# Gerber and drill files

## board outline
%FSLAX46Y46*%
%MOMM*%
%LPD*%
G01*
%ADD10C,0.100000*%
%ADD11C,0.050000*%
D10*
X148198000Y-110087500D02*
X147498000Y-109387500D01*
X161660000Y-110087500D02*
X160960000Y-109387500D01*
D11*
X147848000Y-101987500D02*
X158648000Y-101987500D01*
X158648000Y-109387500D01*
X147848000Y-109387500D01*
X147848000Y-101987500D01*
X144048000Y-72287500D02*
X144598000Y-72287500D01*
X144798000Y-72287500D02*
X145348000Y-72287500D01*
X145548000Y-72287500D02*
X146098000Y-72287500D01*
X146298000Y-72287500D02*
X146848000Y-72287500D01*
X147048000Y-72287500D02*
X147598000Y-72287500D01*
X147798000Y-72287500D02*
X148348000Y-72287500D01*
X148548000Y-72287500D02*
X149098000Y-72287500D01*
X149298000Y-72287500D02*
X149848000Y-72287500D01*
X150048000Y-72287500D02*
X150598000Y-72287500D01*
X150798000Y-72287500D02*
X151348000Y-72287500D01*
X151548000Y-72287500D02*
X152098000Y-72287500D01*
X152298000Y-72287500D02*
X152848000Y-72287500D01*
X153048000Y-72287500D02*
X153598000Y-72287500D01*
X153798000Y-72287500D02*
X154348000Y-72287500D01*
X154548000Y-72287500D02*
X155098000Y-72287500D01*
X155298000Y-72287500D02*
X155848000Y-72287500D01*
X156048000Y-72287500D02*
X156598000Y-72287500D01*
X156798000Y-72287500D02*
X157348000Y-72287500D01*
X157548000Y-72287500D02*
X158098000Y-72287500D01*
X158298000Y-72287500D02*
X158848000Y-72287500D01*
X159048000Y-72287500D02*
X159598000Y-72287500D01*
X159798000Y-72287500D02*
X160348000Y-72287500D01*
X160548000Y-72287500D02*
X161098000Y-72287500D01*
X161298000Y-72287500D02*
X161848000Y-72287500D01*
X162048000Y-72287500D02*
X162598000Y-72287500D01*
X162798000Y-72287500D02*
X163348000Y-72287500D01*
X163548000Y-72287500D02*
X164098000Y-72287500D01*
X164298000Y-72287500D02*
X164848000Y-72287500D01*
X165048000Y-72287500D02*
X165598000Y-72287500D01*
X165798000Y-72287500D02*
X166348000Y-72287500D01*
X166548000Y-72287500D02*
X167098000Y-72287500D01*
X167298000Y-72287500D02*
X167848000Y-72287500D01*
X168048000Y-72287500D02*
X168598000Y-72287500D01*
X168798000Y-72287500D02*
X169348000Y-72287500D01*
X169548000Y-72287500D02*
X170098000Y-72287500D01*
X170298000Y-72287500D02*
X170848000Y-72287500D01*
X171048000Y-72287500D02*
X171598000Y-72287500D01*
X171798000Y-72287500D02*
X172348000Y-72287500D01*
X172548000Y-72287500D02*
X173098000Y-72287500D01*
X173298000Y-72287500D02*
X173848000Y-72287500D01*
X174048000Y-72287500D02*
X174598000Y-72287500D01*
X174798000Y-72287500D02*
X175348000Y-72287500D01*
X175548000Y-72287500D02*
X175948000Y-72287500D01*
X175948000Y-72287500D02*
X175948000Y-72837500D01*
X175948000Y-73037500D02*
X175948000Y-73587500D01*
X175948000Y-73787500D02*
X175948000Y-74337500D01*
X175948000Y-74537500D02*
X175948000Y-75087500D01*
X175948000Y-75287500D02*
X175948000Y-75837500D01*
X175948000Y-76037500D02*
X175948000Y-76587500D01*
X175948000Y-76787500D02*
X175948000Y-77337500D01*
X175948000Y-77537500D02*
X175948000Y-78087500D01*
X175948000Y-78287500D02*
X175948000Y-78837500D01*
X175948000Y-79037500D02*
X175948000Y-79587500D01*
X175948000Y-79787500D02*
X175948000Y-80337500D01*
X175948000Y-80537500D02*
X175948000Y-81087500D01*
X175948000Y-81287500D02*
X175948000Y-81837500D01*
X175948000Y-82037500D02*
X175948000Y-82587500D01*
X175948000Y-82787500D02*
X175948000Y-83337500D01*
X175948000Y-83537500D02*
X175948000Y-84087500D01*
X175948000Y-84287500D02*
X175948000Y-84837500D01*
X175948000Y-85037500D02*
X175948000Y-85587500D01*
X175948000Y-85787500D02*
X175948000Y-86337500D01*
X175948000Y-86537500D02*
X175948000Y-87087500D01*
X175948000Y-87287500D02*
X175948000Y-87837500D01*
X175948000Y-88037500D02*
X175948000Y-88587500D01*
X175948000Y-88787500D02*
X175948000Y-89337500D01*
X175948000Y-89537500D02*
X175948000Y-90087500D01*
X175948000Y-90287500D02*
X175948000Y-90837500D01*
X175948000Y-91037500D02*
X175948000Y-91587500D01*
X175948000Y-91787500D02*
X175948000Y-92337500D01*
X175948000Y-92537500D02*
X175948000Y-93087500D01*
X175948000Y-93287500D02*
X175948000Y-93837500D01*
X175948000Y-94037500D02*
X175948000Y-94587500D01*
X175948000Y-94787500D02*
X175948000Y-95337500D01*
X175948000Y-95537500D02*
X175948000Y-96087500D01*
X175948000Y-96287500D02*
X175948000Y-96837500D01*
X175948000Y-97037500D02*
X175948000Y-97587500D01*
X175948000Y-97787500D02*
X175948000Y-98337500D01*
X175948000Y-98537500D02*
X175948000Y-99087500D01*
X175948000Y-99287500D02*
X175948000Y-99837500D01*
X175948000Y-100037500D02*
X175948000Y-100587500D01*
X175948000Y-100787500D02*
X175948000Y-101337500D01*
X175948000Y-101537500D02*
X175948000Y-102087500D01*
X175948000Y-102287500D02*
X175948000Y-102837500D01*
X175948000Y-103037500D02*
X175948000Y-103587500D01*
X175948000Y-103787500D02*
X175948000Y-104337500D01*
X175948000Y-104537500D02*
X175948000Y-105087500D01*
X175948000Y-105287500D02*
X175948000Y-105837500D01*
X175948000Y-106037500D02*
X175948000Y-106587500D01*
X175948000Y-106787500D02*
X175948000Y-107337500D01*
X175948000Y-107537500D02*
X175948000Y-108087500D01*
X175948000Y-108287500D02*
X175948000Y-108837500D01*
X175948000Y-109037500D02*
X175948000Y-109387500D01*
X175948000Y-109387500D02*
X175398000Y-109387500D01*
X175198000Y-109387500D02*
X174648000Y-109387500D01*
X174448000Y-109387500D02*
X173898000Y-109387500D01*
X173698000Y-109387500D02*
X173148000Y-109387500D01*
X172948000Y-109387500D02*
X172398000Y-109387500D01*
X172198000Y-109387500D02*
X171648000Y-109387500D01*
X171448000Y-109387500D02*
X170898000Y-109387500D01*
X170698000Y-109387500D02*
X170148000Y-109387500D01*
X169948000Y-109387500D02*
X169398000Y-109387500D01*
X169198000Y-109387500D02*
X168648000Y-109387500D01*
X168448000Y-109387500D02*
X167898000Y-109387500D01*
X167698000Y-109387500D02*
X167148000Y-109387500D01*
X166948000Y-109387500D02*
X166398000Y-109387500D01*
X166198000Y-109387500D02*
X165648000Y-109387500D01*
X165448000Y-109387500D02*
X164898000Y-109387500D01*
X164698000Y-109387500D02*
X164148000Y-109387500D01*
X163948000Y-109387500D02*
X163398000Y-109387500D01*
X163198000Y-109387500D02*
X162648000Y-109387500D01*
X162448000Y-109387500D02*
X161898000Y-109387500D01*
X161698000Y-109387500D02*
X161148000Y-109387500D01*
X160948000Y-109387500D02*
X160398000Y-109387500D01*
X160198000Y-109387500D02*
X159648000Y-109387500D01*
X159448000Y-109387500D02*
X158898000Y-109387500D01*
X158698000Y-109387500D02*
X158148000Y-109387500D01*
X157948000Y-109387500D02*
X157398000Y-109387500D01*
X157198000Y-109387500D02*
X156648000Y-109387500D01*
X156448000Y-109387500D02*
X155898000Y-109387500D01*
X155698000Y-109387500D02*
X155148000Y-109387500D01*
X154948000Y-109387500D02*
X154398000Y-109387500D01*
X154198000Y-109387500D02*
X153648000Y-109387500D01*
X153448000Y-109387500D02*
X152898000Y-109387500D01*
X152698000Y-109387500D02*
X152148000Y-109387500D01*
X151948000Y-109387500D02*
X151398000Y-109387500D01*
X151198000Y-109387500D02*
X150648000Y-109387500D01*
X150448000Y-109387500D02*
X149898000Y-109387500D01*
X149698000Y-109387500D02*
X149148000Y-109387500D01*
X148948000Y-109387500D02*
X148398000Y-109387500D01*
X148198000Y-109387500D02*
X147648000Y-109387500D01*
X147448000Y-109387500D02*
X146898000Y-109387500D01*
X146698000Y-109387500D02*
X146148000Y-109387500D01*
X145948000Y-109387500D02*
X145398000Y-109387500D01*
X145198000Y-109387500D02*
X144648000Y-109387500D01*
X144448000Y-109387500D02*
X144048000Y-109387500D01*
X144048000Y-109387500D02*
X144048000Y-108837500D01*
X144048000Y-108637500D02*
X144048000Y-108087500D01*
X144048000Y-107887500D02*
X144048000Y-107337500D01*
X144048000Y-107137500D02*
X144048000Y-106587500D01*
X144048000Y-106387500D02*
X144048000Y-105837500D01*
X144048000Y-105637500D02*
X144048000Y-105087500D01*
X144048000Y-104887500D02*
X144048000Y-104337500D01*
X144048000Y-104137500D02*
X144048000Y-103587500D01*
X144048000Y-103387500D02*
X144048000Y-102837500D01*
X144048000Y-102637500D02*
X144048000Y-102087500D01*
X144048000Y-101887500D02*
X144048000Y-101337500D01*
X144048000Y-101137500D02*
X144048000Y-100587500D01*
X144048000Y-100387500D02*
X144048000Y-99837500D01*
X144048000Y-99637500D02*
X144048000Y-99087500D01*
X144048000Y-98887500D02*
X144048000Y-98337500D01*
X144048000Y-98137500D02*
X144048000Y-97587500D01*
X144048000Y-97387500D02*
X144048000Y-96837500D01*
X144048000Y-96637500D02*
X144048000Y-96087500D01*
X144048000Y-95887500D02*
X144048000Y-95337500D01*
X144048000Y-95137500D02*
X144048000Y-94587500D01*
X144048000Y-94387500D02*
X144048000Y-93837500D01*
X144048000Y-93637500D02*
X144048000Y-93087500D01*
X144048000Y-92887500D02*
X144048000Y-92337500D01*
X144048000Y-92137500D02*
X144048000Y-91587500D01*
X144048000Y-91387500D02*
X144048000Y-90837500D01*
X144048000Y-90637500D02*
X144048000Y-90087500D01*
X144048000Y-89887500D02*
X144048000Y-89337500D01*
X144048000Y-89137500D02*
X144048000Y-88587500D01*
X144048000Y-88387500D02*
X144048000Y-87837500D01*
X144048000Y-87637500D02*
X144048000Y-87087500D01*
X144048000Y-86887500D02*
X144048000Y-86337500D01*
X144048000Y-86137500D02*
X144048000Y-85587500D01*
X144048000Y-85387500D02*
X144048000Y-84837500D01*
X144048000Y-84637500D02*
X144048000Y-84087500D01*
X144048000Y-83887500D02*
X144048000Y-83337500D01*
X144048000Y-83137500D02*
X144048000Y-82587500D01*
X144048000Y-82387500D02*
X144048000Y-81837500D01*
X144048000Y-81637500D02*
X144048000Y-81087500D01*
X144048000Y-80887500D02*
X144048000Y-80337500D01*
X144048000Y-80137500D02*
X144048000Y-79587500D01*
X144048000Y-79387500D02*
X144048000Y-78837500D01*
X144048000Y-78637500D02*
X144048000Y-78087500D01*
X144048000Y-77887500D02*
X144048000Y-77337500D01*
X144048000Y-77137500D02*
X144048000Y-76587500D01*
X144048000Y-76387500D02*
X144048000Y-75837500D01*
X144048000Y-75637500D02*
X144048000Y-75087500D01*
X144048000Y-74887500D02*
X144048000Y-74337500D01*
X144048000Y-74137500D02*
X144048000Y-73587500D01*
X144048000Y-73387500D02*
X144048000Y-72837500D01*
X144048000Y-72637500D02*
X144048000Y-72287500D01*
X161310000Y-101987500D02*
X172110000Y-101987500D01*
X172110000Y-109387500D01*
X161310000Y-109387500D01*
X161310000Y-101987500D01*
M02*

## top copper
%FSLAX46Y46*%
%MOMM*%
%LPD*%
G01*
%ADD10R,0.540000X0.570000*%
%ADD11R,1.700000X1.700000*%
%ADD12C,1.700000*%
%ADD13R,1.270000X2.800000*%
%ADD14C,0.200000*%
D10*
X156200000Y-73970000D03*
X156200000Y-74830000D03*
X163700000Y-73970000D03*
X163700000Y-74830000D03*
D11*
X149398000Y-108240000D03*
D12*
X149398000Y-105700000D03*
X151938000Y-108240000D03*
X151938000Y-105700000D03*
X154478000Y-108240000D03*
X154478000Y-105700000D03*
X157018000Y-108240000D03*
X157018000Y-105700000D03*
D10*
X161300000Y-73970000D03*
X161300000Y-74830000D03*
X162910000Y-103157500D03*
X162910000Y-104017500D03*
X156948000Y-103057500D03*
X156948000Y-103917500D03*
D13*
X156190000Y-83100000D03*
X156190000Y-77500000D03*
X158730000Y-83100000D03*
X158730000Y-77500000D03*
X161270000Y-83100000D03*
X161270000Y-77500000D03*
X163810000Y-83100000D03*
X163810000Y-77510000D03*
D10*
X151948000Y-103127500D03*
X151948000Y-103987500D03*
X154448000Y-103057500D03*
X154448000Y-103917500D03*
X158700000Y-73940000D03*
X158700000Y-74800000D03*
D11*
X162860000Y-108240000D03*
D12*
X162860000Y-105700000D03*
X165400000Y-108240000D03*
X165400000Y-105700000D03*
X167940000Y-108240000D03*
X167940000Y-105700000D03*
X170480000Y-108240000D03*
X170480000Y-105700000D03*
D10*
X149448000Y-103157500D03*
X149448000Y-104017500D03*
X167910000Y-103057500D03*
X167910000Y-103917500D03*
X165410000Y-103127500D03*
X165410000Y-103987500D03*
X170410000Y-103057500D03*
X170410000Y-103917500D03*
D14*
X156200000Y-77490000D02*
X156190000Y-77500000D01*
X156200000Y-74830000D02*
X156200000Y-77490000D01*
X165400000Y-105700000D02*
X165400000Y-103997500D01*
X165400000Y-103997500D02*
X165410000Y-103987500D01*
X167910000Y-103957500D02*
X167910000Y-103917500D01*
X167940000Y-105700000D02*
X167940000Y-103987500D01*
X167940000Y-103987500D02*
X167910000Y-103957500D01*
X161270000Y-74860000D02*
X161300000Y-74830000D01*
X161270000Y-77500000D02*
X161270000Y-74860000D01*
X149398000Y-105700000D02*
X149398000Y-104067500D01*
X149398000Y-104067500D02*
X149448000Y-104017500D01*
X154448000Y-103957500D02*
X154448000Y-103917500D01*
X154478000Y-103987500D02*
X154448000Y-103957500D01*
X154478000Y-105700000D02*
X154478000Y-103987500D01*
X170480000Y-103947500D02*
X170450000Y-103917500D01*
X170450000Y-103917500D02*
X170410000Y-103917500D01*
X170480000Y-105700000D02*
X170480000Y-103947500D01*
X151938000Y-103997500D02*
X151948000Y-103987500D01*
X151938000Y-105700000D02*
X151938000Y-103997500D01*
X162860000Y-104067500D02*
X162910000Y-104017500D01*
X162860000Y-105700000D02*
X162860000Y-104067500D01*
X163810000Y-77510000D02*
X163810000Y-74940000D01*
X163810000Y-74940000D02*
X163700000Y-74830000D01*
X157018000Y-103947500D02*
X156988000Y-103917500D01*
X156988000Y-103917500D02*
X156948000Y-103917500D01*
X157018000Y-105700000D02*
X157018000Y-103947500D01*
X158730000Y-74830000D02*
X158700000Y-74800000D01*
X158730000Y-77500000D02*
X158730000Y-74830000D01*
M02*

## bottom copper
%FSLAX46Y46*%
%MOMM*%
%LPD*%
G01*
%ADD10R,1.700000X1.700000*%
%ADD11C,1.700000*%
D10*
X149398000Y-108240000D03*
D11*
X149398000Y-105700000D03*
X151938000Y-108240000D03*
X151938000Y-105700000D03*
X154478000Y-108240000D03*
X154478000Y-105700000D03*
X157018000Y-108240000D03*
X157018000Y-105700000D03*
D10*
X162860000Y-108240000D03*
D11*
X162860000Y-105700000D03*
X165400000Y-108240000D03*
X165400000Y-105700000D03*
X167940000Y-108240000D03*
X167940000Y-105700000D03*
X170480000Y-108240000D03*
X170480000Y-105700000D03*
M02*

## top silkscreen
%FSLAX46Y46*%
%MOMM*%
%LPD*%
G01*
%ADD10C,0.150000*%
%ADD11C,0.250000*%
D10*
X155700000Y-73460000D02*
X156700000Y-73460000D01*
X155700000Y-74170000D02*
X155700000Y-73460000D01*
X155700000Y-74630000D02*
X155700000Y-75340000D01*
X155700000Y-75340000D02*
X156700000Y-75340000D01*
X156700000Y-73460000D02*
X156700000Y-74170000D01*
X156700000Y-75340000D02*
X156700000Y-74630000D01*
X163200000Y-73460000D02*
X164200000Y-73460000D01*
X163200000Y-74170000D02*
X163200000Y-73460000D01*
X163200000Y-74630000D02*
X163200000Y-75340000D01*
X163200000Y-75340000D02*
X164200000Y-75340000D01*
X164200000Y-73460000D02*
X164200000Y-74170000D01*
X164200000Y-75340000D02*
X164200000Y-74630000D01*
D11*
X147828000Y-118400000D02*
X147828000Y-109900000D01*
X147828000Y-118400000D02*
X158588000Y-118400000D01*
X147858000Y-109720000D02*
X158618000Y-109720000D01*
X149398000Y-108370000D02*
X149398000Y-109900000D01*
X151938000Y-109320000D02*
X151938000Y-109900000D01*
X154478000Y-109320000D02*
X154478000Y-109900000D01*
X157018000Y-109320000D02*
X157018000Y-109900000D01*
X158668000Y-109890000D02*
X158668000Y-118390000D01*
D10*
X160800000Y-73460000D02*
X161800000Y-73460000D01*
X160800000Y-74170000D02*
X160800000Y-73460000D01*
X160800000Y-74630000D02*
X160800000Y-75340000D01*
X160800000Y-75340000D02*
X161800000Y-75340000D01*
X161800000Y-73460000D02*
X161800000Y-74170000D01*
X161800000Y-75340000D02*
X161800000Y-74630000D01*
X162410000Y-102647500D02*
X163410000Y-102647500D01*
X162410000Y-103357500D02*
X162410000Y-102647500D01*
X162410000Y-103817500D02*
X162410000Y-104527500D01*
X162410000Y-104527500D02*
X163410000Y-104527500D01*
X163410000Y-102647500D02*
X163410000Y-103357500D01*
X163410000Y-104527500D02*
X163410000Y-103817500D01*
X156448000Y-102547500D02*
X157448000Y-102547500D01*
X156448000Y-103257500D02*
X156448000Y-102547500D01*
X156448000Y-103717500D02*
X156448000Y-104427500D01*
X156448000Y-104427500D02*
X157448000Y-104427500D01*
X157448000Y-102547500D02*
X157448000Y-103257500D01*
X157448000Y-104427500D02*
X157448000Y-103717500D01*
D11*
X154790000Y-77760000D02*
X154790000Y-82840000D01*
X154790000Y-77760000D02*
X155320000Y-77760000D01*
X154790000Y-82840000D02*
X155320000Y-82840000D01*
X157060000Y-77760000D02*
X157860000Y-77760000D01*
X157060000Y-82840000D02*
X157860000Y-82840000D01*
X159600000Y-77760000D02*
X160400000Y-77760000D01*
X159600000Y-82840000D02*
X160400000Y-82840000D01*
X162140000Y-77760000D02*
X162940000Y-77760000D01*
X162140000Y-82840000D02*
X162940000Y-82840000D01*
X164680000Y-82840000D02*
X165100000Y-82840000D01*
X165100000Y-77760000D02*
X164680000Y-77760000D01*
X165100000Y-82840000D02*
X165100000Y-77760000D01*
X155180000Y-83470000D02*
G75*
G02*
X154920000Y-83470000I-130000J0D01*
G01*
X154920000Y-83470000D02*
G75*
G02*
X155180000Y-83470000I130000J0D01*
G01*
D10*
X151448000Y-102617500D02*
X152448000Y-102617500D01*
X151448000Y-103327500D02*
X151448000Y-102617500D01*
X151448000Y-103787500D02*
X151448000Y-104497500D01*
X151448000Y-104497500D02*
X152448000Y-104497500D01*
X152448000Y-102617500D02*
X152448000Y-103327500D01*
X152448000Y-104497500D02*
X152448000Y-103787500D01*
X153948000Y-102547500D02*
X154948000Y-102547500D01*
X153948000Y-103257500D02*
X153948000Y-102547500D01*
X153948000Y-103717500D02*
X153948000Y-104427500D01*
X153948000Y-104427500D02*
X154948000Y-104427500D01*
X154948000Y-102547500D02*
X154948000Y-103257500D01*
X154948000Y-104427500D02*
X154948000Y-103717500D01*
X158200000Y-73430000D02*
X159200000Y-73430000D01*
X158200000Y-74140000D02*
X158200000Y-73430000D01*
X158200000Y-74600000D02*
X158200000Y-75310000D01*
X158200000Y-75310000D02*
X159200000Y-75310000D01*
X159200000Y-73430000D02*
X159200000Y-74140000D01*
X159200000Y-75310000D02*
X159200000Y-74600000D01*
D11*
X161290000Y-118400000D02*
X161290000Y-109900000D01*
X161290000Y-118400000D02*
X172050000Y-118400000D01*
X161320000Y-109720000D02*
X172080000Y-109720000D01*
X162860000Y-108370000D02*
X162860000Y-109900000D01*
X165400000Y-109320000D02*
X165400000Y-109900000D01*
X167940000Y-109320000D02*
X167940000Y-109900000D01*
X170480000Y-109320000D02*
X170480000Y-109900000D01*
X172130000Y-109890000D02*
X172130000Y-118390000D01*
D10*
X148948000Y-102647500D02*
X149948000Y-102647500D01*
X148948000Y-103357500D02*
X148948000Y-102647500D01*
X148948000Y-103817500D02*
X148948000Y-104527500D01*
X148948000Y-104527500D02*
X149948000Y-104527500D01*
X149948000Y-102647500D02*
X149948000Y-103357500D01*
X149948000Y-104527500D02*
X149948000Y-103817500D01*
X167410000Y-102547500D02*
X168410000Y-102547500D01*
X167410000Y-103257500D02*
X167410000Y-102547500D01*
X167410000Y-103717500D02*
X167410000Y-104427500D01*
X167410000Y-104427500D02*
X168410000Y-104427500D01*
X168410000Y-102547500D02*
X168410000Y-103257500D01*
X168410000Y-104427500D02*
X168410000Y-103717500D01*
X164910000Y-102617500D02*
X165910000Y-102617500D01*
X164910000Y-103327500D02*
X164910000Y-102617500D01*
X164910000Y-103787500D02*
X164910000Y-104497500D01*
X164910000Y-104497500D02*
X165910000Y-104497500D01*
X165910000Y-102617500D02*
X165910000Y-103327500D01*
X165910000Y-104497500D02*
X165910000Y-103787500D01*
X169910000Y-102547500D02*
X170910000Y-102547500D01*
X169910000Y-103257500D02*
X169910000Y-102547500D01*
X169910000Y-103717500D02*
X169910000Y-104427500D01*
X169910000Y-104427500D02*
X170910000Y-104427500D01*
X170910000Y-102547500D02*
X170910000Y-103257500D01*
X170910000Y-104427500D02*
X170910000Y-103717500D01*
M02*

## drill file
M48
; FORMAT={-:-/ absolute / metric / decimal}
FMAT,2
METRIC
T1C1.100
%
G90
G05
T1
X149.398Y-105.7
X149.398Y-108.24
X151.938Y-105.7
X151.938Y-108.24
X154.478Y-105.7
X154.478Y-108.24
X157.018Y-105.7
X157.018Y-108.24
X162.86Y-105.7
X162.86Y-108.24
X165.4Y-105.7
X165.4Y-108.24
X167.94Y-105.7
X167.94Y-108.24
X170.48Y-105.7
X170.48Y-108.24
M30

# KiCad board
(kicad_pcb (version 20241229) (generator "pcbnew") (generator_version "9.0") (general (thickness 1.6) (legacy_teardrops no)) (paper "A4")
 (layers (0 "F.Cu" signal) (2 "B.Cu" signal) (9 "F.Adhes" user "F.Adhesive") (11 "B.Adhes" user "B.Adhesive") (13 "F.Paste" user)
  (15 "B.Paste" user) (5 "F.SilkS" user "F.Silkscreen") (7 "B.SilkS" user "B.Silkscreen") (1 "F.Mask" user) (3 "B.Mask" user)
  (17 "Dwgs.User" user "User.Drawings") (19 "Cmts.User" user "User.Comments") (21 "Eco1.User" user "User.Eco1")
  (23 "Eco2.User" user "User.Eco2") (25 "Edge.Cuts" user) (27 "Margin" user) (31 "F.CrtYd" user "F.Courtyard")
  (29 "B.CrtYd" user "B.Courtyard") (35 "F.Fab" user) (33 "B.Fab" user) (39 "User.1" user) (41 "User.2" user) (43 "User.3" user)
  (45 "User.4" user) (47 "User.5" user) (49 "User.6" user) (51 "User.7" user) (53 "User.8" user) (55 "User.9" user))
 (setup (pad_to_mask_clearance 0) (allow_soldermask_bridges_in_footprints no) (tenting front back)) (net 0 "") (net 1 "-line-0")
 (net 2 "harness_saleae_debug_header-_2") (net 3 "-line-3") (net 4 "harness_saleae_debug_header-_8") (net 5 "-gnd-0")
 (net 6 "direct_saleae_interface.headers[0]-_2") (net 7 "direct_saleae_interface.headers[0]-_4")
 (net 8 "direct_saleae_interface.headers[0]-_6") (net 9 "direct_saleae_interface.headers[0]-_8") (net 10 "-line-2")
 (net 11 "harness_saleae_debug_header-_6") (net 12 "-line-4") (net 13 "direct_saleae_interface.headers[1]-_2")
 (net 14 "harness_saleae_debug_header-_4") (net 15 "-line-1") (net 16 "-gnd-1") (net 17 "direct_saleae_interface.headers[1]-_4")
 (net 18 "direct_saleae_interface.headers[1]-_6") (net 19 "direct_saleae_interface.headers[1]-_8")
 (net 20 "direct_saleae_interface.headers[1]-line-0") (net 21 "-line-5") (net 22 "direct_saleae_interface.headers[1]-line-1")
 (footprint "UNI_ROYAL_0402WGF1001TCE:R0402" (layer "F.Cu") (at 156.2 74.4 -90)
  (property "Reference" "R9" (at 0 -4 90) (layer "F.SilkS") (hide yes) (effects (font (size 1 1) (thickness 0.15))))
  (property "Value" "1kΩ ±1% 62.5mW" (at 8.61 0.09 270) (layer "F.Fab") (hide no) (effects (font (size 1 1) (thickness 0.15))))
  (fp_line (start -0.94 0.5) (end -0.94 -0.5) (stroke (width 0.15) (type solid)) (layer "F.SilkS"))
  (fp_line (start -0.23 0.5) (end -0.94 0.5) (stroke (width 0.15) (type solid)) (layer "F.SilkS"))
  (fp_line (start 0.23 0.5) (end 0.94 0.5) (stroke (width 0.15) (type solid)) (layer "F.SilkS"))
  (fp_line (start 0.94 0.5) (end 0.94 -0.5) (stroke (width 0.15) (type solid)) (layer "F.SilkS"))
  (fp_line (start -0.94 -0.5) (end -0.23 -0.5) (stroke (width 0.15) (type solid)) (layer "F.SilkS"))
  (fp_line (start 0.94 -0.5) (end 0.23 -0.5) (stroke (width 0.15) (type solid)) (layer "F.SilkS"))
  (pad "1" smd rect (at -0.43 0 270) (size 0.57 0.54) (layers "F.Cu" "F.Mask" "F.Paste") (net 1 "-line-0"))
  (pad "2" smd rect (at 0.43 0 270) (size 0.57 0.54) (layers "F.Cu" "F.Mask" "F.Paste") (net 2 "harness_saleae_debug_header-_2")))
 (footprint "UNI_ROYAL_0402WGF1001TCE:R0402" (layer "F.Cu") (at 163.7 74.4 -90)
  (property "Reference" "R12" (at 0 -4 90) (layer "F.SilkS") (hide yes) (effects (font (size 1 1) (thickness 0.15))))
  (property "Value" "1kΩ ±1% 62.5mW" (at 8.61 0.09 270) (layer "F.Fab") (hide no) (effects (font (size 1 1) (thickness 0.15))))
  (fp_line (start -0.94 0.5) (end -0.94 -0.5) (stroke (width 0.15) (type solid)) (layer "F.SilkS"))
  (fp_line (start -0.23 0.5) (end -0.94 0.5) (stroke (width 0.15) (type solid)) (layer "F.SilkS"))
  (fp_line (start 0.23 0.5) (end 0.94 0.5) (stroke (width 0.15) (type solid)) (layer "F.SilkS"))
  (fp_line (start 0.94 0.5) (end 0.94 -0.5) (stroke (width 0.15) (type solid)) (layer "F.SilkS"))
  (fp_line (start -0.94 -0.5) (end -0.23 -0.5) (stroke (width 0.15) (type solid)) (layer "F.SilkS"))
  (fp_line (start 0.94 -0.5) (end 0.23 -0.5) (stroke (width 0.15) (type solid)) (layer "F.SilkS"))
  (pad "1" smd rect (at -0.43 0 270) (size 0.57 0.54) (layers "F.Cu" "F.Mask" "F.Paste") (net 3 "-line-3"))
  (pad "2" smd rect (at 0.43 0 270) (size 0.57 0.54) (layers "F.Cu" "F.Mask" "F.Paste") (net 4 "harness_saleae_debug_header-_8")))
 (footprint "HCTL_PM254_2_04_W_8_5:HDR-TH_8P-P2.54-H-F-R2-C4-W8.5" (layer "F.Cu") (at 153.208 106.97 0)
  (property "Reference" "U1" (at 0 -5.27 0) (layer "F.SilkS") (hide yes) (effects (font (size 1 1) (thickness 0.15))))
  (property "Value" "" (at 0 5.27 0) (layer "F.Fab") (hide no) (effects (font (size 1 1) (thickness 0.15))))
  (fp_line (start -5.38 11.43) (end -5.38 2.93) (stroke (width 0.25) (type solid)) (layer "F.SilkS"))
  (fp_line (start -5.38 11.43) (end 5.38 11.43) (stroke (width 0.25) (type solid)) (layer "F.SilkS"))
  (fp_line (start -5.35 2.75) (end 5.41 2.75) (stroke (width 0.25) (type solid)) (layer "F.SilkS"))
  (fp_line (start -3.81 1.4) (end -3.81 2.93) (stroke (width 0.25) (type solid)) (layer "F.SilkS"))
  (fp_line (start -1.27 2.35) (end -1.27 2.93) (stroke (width 0.25) (type solid)) (layer "F.SilkS"))
  (fp_line (start 1.27 2.35) (end 1.27 2.93) (stroke (width 0.25) (type solid)) (layer "F.SilkS"))
  (fp_line (start 3.81 2.35) (end 3.81 2.93) (stroke (width 0.25) (type solid)) (layer "F.SilkS"))
  (fp_line (start 5.46 2.92) (end 5.46 11.42) (stroke (width 0.25) (type solid)) (layer "F.SilkS"))
  (pad "1" thru_hole rect (at -3.81 1.27 0) (size 1.7 1.7) (drill 1.100023) (layers "*.Cu" "*.Mask") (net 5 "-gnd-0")
   (remove_unused_layers no))
  (pad "2" thru_hole circle (at -3.81 -1.27 0) (size 1.7 1.7) (drill 1.100023) (layers "*.Cu" "*.Mask")
   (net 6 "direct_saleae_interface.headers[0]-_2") (remove_unused_layers no))
  (pad "3" thru_hole circle (at -1.27 1.27 0) (size 1.7 1.7) (drill 1.100023) (layers "*.Cu" "*.Mask") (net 5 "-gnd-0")
   (remove_unused_layers no))
  (pad "4" thru_hole circle (at -1.27 -1.27 0) (size 1.7 1.7) (drill 1.100023) (layers "*.Cu" "*.Mask")
   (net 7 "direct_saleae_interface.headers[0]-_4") (remove_unused_layers no))
  (pad "5" thru_hole circle (at 1.27 1.27 0) (size 1.7 1.7) (drill 1.100023) (layers "*.Cu" "*.Mask") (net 5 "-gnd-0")
   (remove_unused_layers no))
  (pad "6" thru_hole circle (at 1.27 -1.27 0) (size 1.7 1.7) (drill 1.100023) (layers "*.Cu" "*.Mask")
   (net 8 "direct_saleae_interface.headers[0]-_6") (remove_unused_layers no))
  (pad "7" thru_hole circle (at 3.81 1.27 0) (size 1.7 1.7) (drill 1.100023) (layers "*.Cu" "*.Mask") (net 5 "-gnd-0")
   (remove_unused_layers no))
  (pad "8" thru_hole circle (at 3.81 -1.27 0) (size 1.7 1.7) (drill 1.100023) (layers "*.Cu" "*.Mask")
   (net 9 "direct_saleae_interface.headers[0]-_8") (remove_unused_layers no)))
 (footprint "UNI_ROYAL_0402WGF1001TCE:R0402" (layer "F.Cu") (at 161.3 74.4 -90)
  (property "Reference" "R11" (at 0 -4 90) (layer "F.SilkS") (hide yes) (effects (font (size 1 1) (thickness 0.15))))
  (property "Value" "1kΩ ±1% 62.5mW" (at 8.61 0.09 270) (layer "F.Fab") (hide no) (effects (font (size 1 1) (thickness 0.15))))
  (fp_line (start -0.94 0.5) (end -0.94 -0.5) (stroke (width 0.15) (type solid)) (layer "F.SilkS"))
  (fp_line (start -0.23 0.5) (end -0.94 0.5) (stroke (width 0.15) (type solid)) (layer "F.SilkS"))
  (fp_line (start 0.23 0.5) (end 0.94 0.5) (stroke (width 0.15) (type solid)) (layer "F.SilkS"))
  (fp_line (start 0.94 0.5) (end 0.94 -0.5) (stroke (width 0.15) (type solid)) (layer "F.SilkS"))
  (fp_line (start -0.94 -0.5) (end -0.23 -0.5) (stroke (width 0.15) (type solid)) (layer "F.SilkS"))
  (fp_line (start 0.94 -0.5) (end 0.23 -0.5) (stroke (width 0.15) (type solid)) (layer "F.SilkS"))
  (pad "1" smd rect (at -0.43 0 270) (size 0.57 0.54) (layers "F.Cu" "F.Mask" "F.Paste") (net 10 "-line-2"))
  (pad "2" smd rect (at 0.43 0 270) (size 0.57 0.54) (layers "F.Cu" "F.Mask" "F.Paste") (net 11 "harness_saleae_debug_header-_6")))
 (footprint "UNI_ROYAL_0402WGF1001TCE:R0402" (layer "F.Cu") (at 162.91 103.5875 -90)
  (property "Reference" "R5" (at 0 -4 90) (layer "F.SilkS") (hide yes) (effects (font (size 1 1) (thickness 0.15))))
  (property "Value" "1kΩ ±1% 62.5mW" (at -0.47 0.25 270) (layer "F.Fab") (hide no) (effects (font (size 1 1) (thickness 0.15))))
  (fp_line (start -0.94 0.5) (end -0.94 -0.5) (stroke (width 0.15) (type solid)) (layer "F.SilkS"))
  (fp_line (start -0.23 0.5) (end -0.94 0.5) (stroke (width 0.15) (type solid)) (layer "F.SilkS"))
  (fp_line (start 0.23 0.5) (end 0.94 0.5) (stroke (width 0.15) (type solid)) (layer "F.SilkS"))
  (fp_line (start 0.94 0.5) (end 0.94 -0.5) (stroke (width 0.15) (type solid)) (layer "F.SilkS"))
  (fp_line (start -0.94 -0.5) (end -0.23 -0.5) (stroke (width 0.15) (type solid)) (layer "F.SilkS"))
  (fp_line (start 0.94 -0.5) (end 0.23 -0.5) (stroke (width 0.15) (type solid)) (layer "F.SilkS"))
  (pad "1" smd rect (at -0.43 0 270) (size 0.57 0.54) (layers "F.Cu" "F.Mask" "F.Paste") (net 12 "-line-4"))
  (pad "2" smd rect (at 0.43 0 270) (size 0.57 0.54) (layers "F.Cu" "F.Mask" "F.Paste") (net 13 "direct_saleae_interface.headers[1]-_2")))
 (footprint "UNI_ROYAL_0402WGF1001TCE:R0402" (layer "F.Cu") (at 156.948 103.4875 -90)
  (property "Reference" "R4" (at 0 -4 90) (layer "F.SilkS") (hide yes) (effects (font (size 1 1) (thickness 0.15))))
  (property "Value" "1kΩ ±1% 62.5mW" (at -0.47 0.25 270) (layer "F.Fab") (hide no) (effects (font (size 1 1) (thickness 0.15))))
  (fp_line (start -0.94 0.5) (end -0.94 -0.5) (stroke (width 0.15) (type solid)) (layer "F.SilkS"))
  (fp_line (start -0.23 0.5) (end -0.94 0.5) (stroke (width 0.15) (type solid)) (layer "F.SilkS"))
  (fp_line (start 0.23 0.5) (end 0.94 0.5) (stroke (width 0.15) (type solid)) (layer "F.SilkS"))
  (fp_line (start 0.94 0.5) (end 0.94 -0.5) (stroke (width 0.15) (type solid)) (layer "F.SilkS"))
  (fp_line (start -0.94 -0.5) (end -0.23 -0.5) (stroke (width 0.15) (type solid)) (layer "F.SilkS"))
  (fp_line (start 0.94 -0.5) (end 0.23 -0.5) (stroke (width 0.15) (type solid)) (layer "F.SilkS"))
  (pad "1" smd rect (at -0.43 0 270) (size 0.57 0.54) (layers "F.Cu" "F.Mask" "F.Paste") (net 3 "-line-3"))
  (pad "2" smd rect (at 0.43 0 270) (size 0.57 0.54) (layers "F.Cu" "F.Mask" "F.Paste") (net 9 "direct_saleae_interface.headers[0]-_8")))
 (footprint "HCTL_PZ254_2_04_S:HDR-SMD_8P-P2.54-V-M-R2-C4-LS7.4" (layer "F.Cu") (at 160 80.3 0)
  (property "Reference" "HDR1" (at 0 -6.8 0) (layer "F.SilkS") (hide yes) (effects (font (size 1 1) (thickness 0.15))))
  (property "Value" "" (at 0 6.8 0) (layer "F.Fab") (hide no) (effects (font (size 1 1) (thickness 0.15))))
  (fp_line (start -5.21 -2.54) (end -5.21 2.54) (stroke (width 0.25) (type solid)) (layer "F.SilkS"))
  (fp_line (start -5.21 -2.54) (end -4.68 -2.54) (stroke (width 0.25) (type solid)) (layer "F.SilkS"))
  (fp_line (start -5.21 2.54) (end -4.68 2.54) (stroke (width 0.25) (type solid)) (layer "F.SilkS"))
  (fp_line (start -2.94 -2.54) (end -2.14 -2.54) (stroke (width 0.25) (type solid)) (layer "F.SilkS"))
  (fp_line (start -2.94 2.54) (end -2.14 2.54) (stroke (width 0.25) (type solid)) (layer "F.SilkS"))
  (fp_line (start -0.4 -2.54) (end 0.4 -2.54) (stroke (width 0.25) (type solid)) (layer "F.SilkS"))
  (fp_line (start -0.4 2.54) (end 0.4 2.54) (stroke (width 0.25) (type solid)) (layer "F.SilkS"))
  (fp_line (start 2.14 -2.54) (end 2.94 -2.54) (stroke (width 0.25) (type solid)) (layer "F.SilkS"))
  (fp_line (start 2.14 2.54) (end 2.94 2.54) (stroke (width 0.25) (type solid)) (layer "F.SilkS"))
  (fp_line (start 4.68 2.54) (end 5.1 2.54) (stroke (width 0.25) (type solid)) (layer "F.SilkS"))
  (fp_line (start 5.1 -2.54) (end 4.68 -2.54) (stroke (width 0.25) (type solid)) (layer "F.SilkS"))
  (fp_line (start 5.1 2.54) (end 5.1 -2.54) (stroke (width 0.25) (type solid)) (layer "F.SilkS"))
  (fp_circle (center -4.95 3.17) (end -4.82 3.17) (stroke (width 0.25) (type solid)) (fill no) (layer "F.SilkS"))
  (pad "1" smd rect (at -3.81 2.8 0) (size 1.27 2.8) (layers "F.Cu" "F.Mask" "F.Paste") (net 5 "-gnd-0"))
  (pad "2" smd rect (at -3.81 -2.8 0) (size 1.27 2.8) (layers "F.Cu" "F.Mask" "F.Paste") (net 2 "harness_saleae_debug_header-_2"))
  (pad "3" smd rect (at -1.27 2.8 0) (size 1.27 2.8) (layers "F.Cu" "F.Mask" "F.Paste") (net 5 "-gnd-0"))
  (pad "4" smd rect (at -1.27 -2.8 0) (size 1.27 2.8) (layers "F.Cu" "F.Mask" "F.Paste") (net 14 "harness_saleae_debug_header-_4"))
  (pad "5" smd rect (at 1.27 2.8 0) (size 1.27 2.8) (layers "F.Cu" "F.Mask" "F.Paste") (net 5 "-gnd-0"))
  (pad "6" smd rect (at 1.27 -2.8 0) (size 1.27 2.8) (layers "F.Cu" "F.Mask" "F.Paste") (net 11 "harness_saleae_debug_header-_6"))
  (pad "7" smd rect (at 3.81 2.8 0) (size 1.27 2.8) (layers "F.Cu" "F.Mask" "F.Paste") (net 5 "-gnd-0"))
  (pad "8" smd rect (at 3.81 -2.79 0) (size 1.27 2.8) (layers "F.Cu" "F.Mask" "F.Paste") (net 4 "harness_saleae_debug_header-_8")))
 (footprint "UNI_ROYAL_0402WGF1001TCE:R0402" (layer "F.Cu") (at 151.948 103.5575 -90)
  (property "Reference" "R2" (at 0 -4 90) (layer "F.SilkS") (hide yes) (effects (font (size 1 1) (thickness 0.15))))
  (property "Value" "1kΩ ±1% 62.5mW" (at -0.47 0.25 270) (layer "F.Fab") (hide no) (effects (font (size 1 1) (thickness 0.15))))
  (fp_line (start -0.94 0.5) (end -0.94 -0.5) (stroke (width 0.15) (type solid)) (layer "F.SilkS"))
  (fp_line (start -0.23 0.5) (end -0.94 0.5) (stroke (width 0.15) (type solid)) (layer "F.SilkS"))
  (fp_line (start 0.23 0.5) (end 0.94 0.5) (stroke (width 0.15) (type solid)) (layer "F.SilkS"))
  (fp_line (start 0.94 0.5) (end 0.94 -0.5) (stroke (width 0.15) (type solid)) (layer "F.SilkS"))
  (fp_line (start -0.94 -0.5) (end -0.23 -0.5) (stroke (width 0.15) (type solid)) (layer "F.SilkS"))
  (fp_line (start 0.94 -0.5) (end 0.23 -0.5) (stroke (width 0.15) (type solid)) (layer "F.SilkS"))
  (pad "1" smd rect (at -0.43 0 270) (size 0.57 0.54) (layers "F.Cu" "F.Mask" "F.Paste") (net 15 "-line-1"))
  (pad "2" smd rect (at 0.43 0 270) (size 0.57 0.54) (layers "F.Cu" "F.Mask" "F.Paste") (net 7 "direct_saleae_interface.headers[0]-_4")))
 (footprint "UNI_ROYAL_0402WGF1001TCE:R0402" (layer "F.Cu") (at 154.448 103.4875 -90)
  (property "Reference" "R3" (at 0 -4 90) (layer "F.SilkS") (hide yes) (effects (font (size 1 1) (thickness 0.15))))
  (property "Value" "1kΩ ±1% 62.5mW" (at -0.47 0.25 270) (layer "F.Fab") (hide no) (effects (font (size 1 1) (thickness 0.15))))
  (fp_line (start -0.94 0.5) (end -0.94 -0.5) (stroke (width 0.15) (type solid)) (layer "F.SilkS"))
  (fp_line (start -0.23 0.5) (end -0.94 0.5) (stroke (width 0.15) (type solid)) (layer "F.SilkS"))
  (fp_line (start 0.23 0.5) (end 0.94 0.5) (stroke (width 0.15) (type solid)) (layer "F.SilkS"))
  (fp_line (start 0.94 0.5) (end 0.94 -0.5) (stroke (width 0.15) (type solid)) (layer "F.SilkS"))
  (fp_line (start -0.94 -0.5) (end -0.23 -0.5) (stroke (width 0.15) (type solid)) (layer "F.SilkS"))
  (fp_line (start 0.94 -0.5) (end 0.23 -0.5) (stroke (width 0.15) (type solid)) (layer "F.SilkS"))
  (pad "1" smd rect (at -0.43 0 270) (size 0.57 0.54) (layers "F.Cu" "F.Mask" "F.Paste") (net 10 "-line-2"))
  (pad "2" smd rect (at 0.43 0 270) (size 0.57 0.54) (layers "F.Cu" "F.Mask" "F.Paste") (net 8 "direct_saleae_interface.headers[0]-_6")))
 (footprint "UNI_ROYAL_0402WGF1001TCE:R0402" (layer "F.Cu") (at 158.7 74.37 -90)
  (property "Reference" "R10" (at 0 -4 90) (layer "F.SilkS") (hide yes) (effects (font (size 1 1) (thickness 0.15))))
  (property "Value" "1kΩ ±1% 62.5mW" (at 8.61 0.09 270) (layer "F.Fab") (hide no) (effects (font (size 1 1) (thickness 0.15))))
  (fp_line (start -0.94 0.5) (end -0.94 -0.5) (stroke (width 0.15) (type solid)) (layer "F.SilkS"))
  (fp_line (start -0.23 0.5) (end -0.94 0.5) (stroke (width 0.15) (type solid)) (layer "F.SilkS"))
  (fp_line (start 0.23 0.5) (end 0.94 0.5) (stroke (width 0.15) (type solid)) (layer "F.SilkS"))
  (fp_line (start 0.94 0.5) (end 0.94 -0.5) (stroke (width 0.15) (type solid)) (layer "F.SilkS"))
  (fp_line (start -0.94 -0.5) (end -0.23 -0.5) (stroke (width 0.15) (type solid)) (layer "F.SilkS"))
  (fp_line (start 0.94 -0.5) (end 0.23 -0.5) (stroke (width 0.15) (type solid)) (layer "F.SilkS"))
  (pad "1" smd rect (at -0.43 0 270) (size 0.57 0.54) (layers "F.Cu" "F.Mask" "F.Paste") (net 15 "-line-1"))
  (pad "2" smd rect (at 0.43 0 270) (size 0.57 0.54) (layers "F.Cu" "F.Mask" "F.Paste") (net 14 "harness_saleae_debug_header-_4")))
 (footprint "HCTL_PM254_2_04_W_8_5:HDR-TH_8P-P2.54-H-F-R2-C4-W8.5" (layer "F.Cu") (at 166.67 106.97 0)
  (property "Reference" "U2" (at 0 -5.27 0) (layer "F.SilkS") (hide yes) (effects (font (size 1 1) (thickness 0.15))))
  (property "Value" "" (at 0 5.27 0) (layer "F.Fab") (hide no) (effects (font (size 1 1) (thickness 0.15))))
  (fp_line (start -5.38 11.43) (end -5.38 2.93) (stroke (width 0.25) (type solid)) (layer "F.SilkS"))
  (fp_line (start -5.38 11.43) (end 5.38 11.43) (stroke (width 0.25) (type solid)) (layer "F.SilkS"))
  (fp_line (start -5.35 2.75) (end 5.41 2.75) (stroke (width 0.25) (type solid)) (layer "F.SilkS"))
  (fp_line (start -3.81 1.4) (end -3.81 2.93) (stroke (width 0.25) (type solid)) (layer "F.SilkS"))
  (fp_line (start -1.27 2.35) (end -1.27 2.93) (stroke (width 0.25) (type solid)) (layer "F.SilkS"))
  (fp_line (start 1.27 2.35) (end 1.27 2.93) (stroke (width 0.25) (type solid)) (layer "F.SilkS"))
  (fp_line (start 3.81 2.35) (end 3.81 2.93) (stroke (width 0.25) (type solid)) (layer "F.SilkS"))
  (fp_line (start 5.46 2.92) (end 5.46 11.42) (stroke (width 0.25) (type solid)) (layer "F.SilkS"))
  (pad "1" thru_hole rect (at -3.81 1.27 0) (size 1.7 1.7) (drill 1.100023) (layers "*.Cu" "*.Mask") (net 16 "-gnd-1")
   (remove_unused_layers no))
  (pad "2" thru_hole circle (at -3.81 -1.27 0) (size 1.7 1.7) (drill 1.100023) (layers "*.Cu" "*.Mask")
   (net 13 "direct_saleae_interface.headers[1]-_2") (remove_unused_layers no))
  (pad "3" thru_hole circle (at -1.27 1.27 0) (size 1.7 1.7) (drill 1.100023) (layers "*.Cu" "*.Mask") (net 16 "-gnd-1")
   (remove_unused_layers no))
  (pad "4" thru_hole circle (at -1.27 -1.27 0) (size 1.7 1.7) (drill 1.100023) (layers "*.Cu" "*.Mask")
   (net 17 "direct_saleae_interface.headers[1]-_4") (remove_unused_layers no))
  (pad "5" thru_hole circle (at 1.27 1.27 0) (size 1.7 1.7) (drill 1.100023) (layers "*.Cu" "*.Mask") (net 16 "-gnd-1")
   (remove_unused_layers no))
  (pad "6" thru_hole circle (at 1.27 -1.27 0) (size 1.7 1.7) (drill 1.100023) (layers "*.Cu" "*.Mask")
   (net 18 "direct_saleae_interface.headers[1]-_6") (remove_unused_layers no))
  (pad "7" thru_hole circle (at 3.81 1.27 0) (size 1.7 1.7) (drill 1.100023) (layers "*.Cu" "*.Mask") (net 16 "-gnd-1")
   (remove_unused_layers no))
  (pad "8" thru_hole circle (at 3.81 -1.27 0) (size 1.7 1.7) (drill 1.100023) (layers "*.Cu" "*.Mask")
   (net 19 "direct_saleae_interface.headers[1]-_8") (remove_unused_layers no)))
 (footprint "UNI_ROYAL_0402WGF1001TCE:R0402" (layer "F.Cu") (at 149.448 103.5875 -90)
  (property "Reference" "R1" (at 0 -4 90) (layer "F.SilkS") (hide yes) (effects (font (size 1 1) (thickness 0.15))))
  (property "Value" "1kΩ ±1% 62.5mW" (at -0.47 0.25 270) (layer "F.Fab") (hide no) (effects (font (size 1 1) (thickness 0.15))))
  (fp_line (start -0.94 0.5) (end -0.94 -0.5) (stroke (width 0.15) (type solid)) (layer "F.SilkS"))
  (fp_line (start -0.23 0.5) (end -0.94 0.5) (stroke (width 0.15) (type solid)) (layer "F.SilkS"))
  (fp_line (start 0.23 0.5) (end 0.94 0.5) (stroke (width 0.15) (type solid)) (layer "F.SilkS"))
  (fp_line (start 0.94 0.5) (end 0.94 -0.5) (stroke (width 0.15) (type solid)) (layer "F.SilkS"))
  (fp_line (start -0.94 -0.5) (end -0.23 -0.5) (stroke (width 0.15) (type solid)) (layer "F.SilkS"))
  (fp_line (start 0.94 -0.5) (end 0.23 -0.5) (stroke (width 0.15) (type solid)) (layer "F.SilkS"))
  (pad "1" smd rect (at -0.43 0 270) (size 0.57 0.54) (layers "F.Cu" "F.Mask" "F.Paste") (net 1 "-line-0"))
  (pad "2" smd rect (at 0.43 0 270) (size 0.57 0.54) (layers "F.Cu" "F.Mask" "F.Paste") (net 6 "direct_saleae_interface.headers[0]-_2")))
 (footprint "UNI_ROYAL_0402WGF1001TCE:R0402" (layer "F.Cu") (at 167.91 103.4875 -90)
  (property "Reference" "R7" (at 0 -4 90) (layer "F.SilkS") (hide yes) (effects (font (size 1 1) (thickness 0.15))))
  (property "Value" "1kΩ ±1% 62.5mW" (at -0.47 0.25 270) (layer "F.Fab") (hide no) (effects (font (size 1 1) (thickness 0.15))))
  (fp_line (start -0.94 0.5) (end -0.94 -0.5) (stroke (width 0.15) (type solid)) (layer "F.SilkS"))
  (fp_line (start -0.23 0.5) (end -0.94 0.5) (stroke (width 0.15) (type solid)) (layer "F.SilkS"))
  (fp_line (start 0.23 0.5) (end 0.94 0.5) (stroke (width 0.15) (type solid)) (layer "F.SilkS"))
  (fp_line (start 0.94 0.5) (end 0.94 -0.5) (stroke (width 0.15) (type solid)) (layer "F.SilkS"))
  (fp_line (start -0.94 -0.5) (end -0.23 -0.5) (stroke (width 0.15) (type solid)) (layer "F.SilkS"))
  (fp_line (start 0.94 -0.5) (end 0.23 -0.5) (stroke (width 0.15) (type solid)) (layer "F.SilkS"))
  (pad "1" smd rect (at -0.43 0 270) (size 0.57 0.54) (layers "F.Cu" "F.Mask" "F.Paste")
   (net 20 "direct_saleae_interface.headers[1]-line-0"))
  (pad "2" smd rect (at 0.43 0 270) (size 0.57 0.54) (layers "F.Cu" "F.Mask" "F.Paste") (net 18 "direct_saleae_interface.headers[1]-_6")))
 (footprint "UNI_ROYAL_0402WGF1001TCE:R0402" (layer "F.Cu") (at 165.41 103.5575 -90)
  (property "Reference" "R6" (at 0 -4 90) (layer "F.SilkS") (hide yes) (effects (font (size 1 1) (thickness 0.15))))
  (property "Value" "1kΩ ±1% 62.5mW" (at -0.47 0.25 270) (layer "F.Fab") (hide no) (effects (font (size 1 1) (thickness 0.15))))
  (fp_line (start -0.94 0.5) (end -0.94 -0.5) (stroke (width 0.15) (type solid)) (layer "F.SilkS"))
  (fp_line (start -0.23 0.5) (end -0.94 0.5) (stroke (width 0.15) (type solid)) (layer "F.SilkS"))
  (fp_line (start 0.23 0.5) (end 0.94 0.5) (stroke (width 0.15) (type solid)) (layer "F.SilkS"))
  (fp_line (start 0.94 0.5) (end 0.94 -0.5) (stroke (width 0.15) (type solid)) (layer "F.SilkS"))
  (fp_line (start -0.94 -0.5) (end -0.23 -0.5) (stroke (width 0.15) (type solid)) (layer "F.SilkS"))
  (fp_line (start 0.94 -0.5) (end 0.23 -0.5) (stroke (width 0.15) (type solid)) (layer "F.SilkS"))
  (pad "1" smd rect (at -0.43 0 270) (size 0.57 0.54) (layers "F.Cu" "F.Mask" "F.Paste") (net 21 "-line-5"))
  (pad "2" smd rect (at 0.43 0 270) (size 0.57 0.54) (layers "F.Cu" "F.Mask" "F.Paste") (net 17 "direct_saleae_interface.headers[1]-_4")))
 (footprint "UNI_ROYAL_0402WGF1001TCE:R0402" (layer "F.Cu") (at 170.41 103.4875 -90)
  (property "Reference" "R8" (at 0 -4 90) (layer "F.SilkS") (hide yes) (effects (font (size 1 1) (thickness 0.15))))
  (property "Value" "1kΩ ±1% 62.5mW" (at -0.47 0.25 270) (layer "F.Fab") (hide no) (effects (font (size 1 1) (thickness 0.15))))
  (fp_line (start -0.94 0.5) (end -0.94 -0.5) (stroke (width 0.15) (type solid)) (layer "F.SilkS"))
  (fp_line (start -0.23 0.5) (end -0.94 0.5) (stroke (width 0.15) (type solid)) (layer "F.SilkS"))
  (fp_line (start 0.23 0.5) (end 0.94 0.5) (stroke (width 0.15) (type solid)) (layer "F.SilkS"))
  (fp_line (start 0.94 0.5) (end 0.94 -0.5) (stroke (width 0.15) (type solid)) (layer "F.SilkS"))
  (fp_line (start -0.94 -0.5) (end -0.23 -0.5) (stroke (width 0.15) (type solid)) (layer "F.SilkS"))
  (fp_line (start 0.94 -0.5) (end 0.23 -0.5) (stroke (width 0.15) (type solid)) (layer "F.SilkS"))
  (pad "1" smd rect (at -0.43 0 270) (size 0.57 0.54) (layers "F.Cu" "F.Mask" "F.Paste")
   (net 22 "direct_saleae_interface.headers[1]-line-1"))
  (pad "2" smd rect (at 0.43 0 270) (size 0.57 0.54) (layers "F.Cu" "F.Mask" "F.Paste") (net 19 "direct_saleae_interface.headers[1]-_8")))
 (segment (start 156.2 77.49) (end 156.19 77.5) (width 0.2) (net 2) (layer "F.Cu"))
 (segment (start 156.2 74.83) (end 156.2 77.49) (width 0.2) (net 2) (layer "F.Cu"))
 (segment (start 165.4 105.7) (end 165.4 103.9975) (width 0.2) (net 17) (layer "F.Cu"))
 (segment (start 165.4 103.9975) (end 165.41 103.9875) (width 0.2) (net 17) (layer "F.Cu"))
 (segment (start 167.91 103.9575) (end 167.91 103.9175) (width 0.2) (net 18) (layer "F.Cu"))
 (segment (start 167.94 105.7) (end 167.94 103.9875) (width 0.2) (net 18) (layer "F.Cu"))
 (segment (start 167.94 103.9875) (end 167.91 103.9575) (width 0.2) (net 18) (layer "F.Cu"))
 (segment (start 161.27 74.86) (end 161.3 74.83) (width 0.2) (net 11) (layer "F.Cu"))
 (segment (start 161.27 77.5) (end 161.27 74.86) (width 0.2) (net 11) (layer "F.Cu"))
 (segment (start 149.398 105.7) (end 149.398 104.0675) (width 0.2) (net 6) (layer "F.Cu"))
 (segment (start 149.398 104.0675) (end 149.448 104.0175) (width 0.2) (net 6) (layer "F.Cu"))
 (segment (start 154.448 103.9575) (end 154.448 103.9175) (width 0.2) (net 8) (layer "F.Cu"))
 (segment (start 154.478 103.9875) (end 154.448 103.9575) (width 0.2) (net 8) (layer "F.Cu"))
 (segment (start 154.478 105.7) (end 154.478 103.9875) (width 0.2) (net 8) (layer "F.Cu"))
 (segment (start 170.48 103.9475) (end 170.45 103.9175) (width 0.2) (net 19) (layer "F.Cu"))
 (segment (start 170.45 103.9175) (end 170.41 103.9175) (width 0.2) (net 19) (layer "F.Cu"))
 (segment (start 170.48 105.7) (end 170.48 103.9475) (width 0.2) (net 19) (layer "F.Cu"))
 (segment (start 151.938 103.9975) (end 151.948 103.9875) (width 0.2) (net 7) (layer "F.Cu"))
 (segment (start 151.938 105.7) (end 151.938 103.9975) (width 0.2) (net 7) (layer "F.Cu"))
 (segment (start 162.86 104.0675) (end 162.91 104.0175) (width 0.2) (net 13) (layer "F.Cu"))
 (segment (start 162.86 105.7) (end 162.86 104.0675) (width 0.2) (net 13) (layer "F.Cu"))
 (segment (start 163.81 77.51) (end 163.81 74.94) (width 0.2) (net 4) (layer "F.Cu"))
 (segment (start 163.81 74.94) (end 163.7 74.83) (width 0.2) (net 4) (layer "F.Cu"))
 (segment (start 157.018 103.9475) (end 156.988 103.9175) (width 0.2) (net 9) (layer "F.Cu"))
 (segment (start 156.988 103.9175) (end 156.948 103.9175) (width 0.2) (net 9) (layer "F.Cu"))
 (segment (start 157.018 105.7) (end 157.018 103.9475) (width 0.2) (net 9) (layer "F.Cu"))
 (segment (start 158.73 74.83) (end 158.7 74.8) (width 0.2) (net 14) (layer "F.Cu"))
 (segment (start 158.73 77.5) (end 158.73 74.83) (width 0.2) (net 14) (layer "F.Cu"))
 (gr_line (start 148.198 110.0875) (end 147.498 109.3875) (stroke (width 0.1) (type solid)) (layer "Edge.Cuts"))
 (gr_line (start 161.66 110.0875) (end 160.96 109.3875) (stroke (width 0.1) (type solid)) (layer "Edge.Cuts"))
 (gr_rect (start 147.848 101.9875) (end 158.648 109.3875) (stroke (width 0.05) (type default)) (fill no) (layer "Edge.Cuts"))
 (gr_rect (start 144.048 72.2875) (end 175.948 109.3875) (stroke (width 0.05) (type dash)) (fill no) (layer "Edge.Cuts"))
 (gr_rect (start 161.31 101.9875) (end 172.11 109.3875) (stroke (width 0.05) (type default)) (fill no) (layer "Edge.Cuts")))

